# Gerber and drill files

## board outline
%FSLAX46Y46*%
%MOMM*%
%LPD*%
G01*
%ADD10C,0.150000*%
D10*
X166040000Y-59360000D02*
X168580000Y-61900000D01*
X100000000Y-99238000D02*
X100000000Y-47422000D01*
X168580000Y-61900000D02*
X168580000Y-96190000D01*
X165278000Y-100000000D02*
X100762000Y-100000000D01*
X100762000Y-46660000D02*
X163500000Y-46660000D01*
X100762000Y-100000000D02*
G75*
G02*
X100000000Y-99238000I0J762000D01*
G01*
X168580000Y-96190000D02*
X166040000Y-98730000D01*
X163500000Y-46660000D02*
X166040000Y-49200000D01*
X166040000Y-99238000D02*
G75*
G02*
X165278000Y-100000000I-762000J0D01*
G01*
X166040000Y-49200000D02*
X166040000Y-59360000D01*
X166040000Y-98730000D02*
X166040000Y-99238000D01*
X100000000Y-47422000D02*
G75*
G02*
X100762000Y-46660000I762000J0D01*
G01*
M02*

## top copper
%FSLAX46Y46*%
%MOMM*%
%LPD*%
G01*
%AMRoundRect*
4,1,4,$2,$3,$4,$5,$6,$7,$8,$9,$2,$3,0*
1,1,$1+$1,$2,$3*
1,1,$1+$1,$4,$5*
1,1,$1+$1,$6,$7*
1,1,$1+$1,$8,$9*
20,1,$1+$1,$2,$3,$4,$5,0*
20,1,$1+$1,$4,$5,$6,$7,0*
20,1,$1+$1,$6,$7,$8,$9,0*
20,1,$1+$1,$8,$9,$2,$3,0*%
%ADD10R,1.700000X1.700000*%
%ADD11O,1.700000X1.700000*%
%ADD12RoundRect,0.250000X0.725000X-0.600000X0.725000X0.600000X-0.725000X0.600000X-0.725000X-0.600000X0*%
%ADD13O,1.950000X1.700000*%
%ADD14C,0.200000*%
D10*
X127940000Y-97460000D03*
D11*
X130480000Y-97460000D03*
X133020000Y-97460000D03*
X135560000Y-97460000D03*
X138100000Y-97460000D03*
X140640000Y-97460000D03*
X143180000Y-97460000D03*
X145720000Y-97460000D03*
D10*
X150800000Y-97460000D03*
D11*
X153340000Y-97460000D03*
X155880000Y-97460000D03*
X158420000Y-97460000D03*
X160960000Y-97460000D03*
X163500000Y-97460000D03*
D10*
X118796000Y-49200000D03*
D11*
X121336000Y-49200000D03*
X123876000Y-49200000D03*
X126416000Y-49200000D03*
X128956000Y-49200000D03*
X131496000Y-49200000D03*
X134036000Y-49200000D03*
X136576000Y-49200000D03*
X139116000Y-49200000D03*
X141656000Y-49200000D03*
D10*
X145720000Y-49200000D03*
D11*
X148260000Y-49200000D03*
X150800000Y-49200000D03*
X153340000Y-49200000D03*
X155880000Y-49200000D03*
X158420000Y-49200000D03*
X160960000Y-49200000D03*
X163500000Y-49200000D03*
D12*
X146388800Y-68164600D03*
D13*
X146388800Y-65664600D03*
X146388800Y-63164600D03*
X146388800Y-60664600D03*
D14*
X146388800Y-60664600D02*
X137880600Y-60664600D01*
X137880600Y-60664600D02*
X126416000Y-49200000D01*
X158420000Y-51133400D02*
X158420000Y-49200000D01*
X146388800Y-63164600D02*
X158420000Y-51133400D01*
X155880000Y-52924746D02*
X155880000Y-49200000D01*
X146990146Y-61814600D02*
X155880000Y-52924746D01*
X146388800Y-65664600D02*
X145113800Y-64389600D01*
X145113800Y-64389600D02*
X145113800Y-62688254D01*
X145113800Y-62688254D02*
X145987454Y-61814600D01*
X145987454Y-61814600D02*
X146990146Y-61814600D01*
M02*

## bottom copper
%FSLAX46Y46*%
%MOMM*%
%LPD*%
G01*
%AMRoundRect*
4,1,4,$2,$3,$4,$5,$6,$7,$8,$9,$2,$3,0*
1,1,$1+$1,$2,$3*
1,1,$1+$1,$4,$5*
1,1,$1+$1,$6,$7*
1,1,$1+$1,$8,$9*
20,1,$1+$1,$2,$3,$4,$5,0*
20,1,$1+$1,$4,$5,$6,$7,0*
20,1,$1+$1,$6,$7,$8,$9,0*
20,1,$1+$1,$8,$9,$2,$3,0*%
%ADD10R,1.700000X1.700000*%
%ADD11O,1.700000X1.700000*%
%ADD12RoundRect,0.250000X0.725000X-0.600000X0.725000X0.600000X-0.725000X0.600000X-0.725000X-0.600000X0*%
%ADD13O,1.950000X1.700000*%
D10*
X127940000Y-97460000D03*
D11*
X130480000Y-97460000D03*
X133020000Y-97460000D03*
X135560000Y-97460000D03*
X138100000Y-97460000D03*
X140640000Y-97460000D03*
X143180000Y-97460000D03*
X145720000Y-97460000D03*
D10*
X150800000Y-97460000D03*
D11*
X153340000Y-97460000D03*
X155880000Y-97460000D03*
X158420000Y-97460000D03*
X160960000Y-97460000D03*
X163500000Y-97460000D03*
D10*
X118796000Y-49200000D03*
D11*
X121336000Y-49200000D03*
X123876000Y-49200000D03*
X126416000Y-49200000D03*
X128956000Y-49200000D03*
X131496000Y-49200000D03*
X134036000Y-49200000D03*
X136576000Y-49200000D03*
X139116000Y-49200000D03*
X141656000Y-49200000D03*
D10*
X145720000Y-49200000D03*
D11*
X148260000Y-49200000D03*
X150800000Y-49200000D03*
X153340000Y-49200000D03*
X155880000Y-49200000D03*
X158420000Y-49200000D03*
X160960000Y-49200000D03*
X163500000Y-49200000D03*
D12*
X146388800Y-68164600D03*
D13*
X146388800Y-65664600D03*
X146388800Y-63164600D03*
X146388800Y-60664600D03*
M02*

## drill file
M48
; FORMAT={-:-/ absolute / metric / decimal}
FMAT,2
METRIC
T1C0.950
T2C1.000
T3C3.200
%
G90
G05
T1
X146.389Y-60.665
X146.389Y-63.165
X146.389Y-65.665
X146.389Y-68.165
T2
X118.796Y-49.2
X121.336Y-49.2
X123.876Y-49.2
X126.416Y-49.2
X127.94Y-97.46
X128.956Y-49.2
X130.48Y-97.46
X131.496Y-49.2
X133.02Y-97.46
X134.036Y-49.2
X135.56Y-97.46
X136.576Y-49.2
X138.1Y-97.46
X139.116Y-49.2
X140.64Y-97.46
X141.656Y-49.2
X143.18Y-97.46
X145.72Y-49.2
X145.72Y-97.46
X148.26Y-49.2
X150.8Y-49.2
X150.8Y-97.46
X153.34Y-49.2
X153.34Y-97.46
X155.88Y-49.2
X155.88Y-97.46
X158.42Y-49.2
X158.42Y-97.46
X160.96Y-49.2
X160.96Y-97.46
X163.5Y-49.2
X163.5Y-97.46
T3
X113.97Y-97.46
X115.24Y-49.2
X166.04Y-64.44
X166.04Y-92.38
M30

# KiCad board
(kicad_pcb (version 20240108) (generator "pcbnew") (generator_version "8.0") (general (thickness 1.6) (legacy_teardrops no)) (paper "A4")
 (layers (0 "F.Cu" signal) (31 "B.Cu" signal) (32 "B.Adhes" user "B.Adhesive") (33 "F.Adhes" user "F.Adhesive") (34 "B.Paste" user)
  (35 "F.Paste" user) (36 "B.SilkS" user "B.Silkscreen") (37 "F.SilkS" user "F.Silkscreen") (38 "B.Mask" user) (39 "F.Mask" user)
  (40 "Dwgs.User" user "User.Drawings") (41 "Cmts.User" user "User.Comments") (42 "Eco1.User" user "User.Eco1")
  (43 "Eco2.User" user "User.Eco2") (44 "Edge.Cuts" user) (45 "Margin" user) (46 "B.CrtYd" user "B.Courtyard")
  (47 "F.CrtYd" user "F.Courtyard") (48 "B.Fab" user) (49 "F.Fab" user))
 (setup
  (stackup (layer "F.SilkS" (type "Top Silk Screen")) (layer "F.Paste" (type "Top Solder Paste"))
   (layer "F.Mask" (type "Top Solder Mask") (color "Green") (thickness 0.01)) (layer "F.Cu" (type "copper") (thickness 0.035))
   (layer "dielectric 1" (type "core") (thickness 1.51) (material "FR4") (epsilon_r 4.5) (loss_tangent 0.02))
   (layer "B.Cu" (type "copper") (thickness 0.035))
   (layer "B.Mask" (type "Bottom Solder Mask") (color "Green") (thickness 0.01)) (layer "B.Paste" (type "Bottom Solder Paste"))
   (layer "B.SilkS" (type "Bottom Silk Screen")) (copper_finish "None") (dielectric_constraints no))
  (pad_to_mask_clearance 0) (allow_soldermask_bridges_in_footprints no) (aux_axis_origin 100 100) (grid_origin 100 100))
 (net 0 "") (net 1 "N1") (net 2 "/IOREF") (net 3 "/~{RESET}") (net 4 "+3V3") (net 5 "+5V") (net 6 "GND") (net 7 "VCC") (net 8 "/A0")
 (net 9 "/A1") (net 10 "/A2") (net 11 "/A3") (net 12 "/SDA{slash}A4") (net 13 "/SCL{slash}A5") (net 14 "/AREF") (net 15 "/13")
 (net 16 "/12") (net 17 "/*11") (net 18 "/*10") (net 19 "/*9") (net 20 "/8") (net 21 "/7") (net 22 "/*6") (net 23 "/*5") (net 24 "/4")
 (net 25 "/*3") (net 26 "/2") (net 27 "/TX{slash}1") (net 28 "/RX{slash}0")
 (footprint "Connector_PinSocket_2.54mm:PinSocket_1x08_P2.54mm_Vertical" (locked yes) (layer "F.Cu") (at 127.94 97.46 90)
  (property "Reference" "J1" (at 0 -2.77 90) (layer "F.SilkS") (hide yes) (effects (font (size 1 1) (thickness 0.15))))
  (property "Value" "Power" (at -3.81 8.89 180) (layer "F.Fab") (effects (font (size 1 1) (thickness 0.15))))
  (pad "1" thru_hole rect (at 0 0 90) (size 1.7 1.7) (drill 1) (layers "*.Cu" "*.Mask") (remove_unused_layers no) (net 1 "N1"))
  (pad "2" thru_hole oval (at 0 2.54 90) (size 1.7 1.7) (drill 1) (layers "*.Cu" "*.Mask") (remove_unused_layers no) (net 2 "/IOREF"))
  (pad "3" thru_hole oval (at 0 5.08 90) (size 1.7 1.7) (drill 1) (layers "*.Cu" "*.Mask") (remove_unused_layers no) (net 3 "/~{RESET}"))
  (pad "4" thru_hole oval (at 0 7.62 90) (size 1.7 1.7) (drill 1) (layers "*.Cu" "*.Mask") (remove_unused_layers no) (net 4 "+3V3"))
  (pad "5" thru_hole oval (at 0 10.16 90) (size 1.7 1.7) (drill 1) (layers "*.Cu" "*.Mask") (remove_unused_layers no) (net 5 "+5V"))
  (pad "6" thru_hole oval (at 0 12.7 90) (size 1.7 1.7) (drill 1) (layers "*.Cu" "*.Mask") (remove_unused_layers no) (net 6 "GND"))
  (pad "7" thru_hole oval (at 0 15.24 90) (size 1.7 1.7) (drill 1) (layers "*.Cu" "*.Mask") (remove_unused_layers no) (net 6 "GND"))
  (pad "8" thru_hole oval (at 0 17.78 90) (size 1.7 1.7) (drill 1) (layers "*.Cu" "*.Mask") (remove_unused_layers no) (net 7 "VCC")))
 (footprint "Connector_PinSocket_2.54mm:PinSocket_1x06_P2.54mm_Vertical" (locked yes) (layer "F.Cu") (at 150.8 97.46 90)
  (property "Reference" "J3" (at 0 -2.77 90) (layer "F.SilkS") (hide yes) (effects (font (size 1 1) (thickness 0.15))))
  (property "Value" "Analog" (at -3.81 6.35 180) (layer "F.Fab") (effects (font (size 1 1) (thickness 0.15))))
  (pad "1" thru_hole rect (at 0 0 90) (size 1.7 1.7) (drill 1) (layers "*.Cu" "*.Mask") (remove_unused_layers no) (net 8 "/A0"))
  (pad "2" thru_hole oval (at 0 2.54 90) (size 1.7 1.7) (drill 1) (layers "*.Cu" "*.Mask") (remove_unused_layers no) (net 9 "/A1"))
  (pad "3" thru_hole oval (at 0 5.08 90) (size 1.7 1.7) (drill 1) (layers "*.Cu" "*.Mask") (remove_unused_layers no) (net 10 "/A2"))
  (pad "4" thru_hole oval (at 0 7.62 90) (size 1.7 1.7) (drill 1) (layers "*.Cu" "*.Mask") (remove_unused_layers no) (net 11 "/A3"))
  (pad "5" thru_hole oval (at 0 10.16 90) (size 1.7 1.7) (drill 1) (layers "*.Cu" "*.Mask") (remove_unused_layers no)
   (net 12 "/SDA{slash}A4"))
  (pad "6" thru_hole oval (at 0 12.7 90) (size 1.7 1.7) (drill 1) (layers "*.Cu" "*.Mask") (remove_unused_layers no)
   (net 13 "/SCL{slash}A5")))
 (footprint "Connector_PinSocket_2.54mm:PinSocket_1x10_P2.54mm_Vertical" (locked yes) (layer "F.Cu") (at 118.796 49.2 90)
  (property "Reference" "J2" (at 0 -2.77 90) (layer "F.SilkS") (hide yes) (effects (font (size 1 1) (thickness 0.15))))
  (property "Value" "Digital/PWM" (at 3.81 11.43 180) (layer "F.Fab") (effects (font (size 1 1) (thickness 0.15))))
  (pad "1" thru_hole rect (at 0 0 90) (size 1.7 1.7) (drill 1) (layers "*.Cu" "*.Mask") (remove_unused_layers no) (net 13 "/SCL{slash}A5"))
  (pad "2" thru_hole oval (at 0 2.54 90) (size 1.7 1.7) (drill 1) (layers "*.Cu" "*.Mask") (remove_unused_layers no)
   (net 12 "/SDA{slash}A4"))
  (pad "3" thru_hole oval (at 0 5.08 90) (size 1.7 1.7) (drill 1) (layers "*.Cu" "*.Mask") (remove_unused_layers no) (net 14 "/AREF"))
  (pad "4" thru_hole oval (at 0 7.62 90) (size 1.7 1.7) (drill 1) (layers "*.Cu" "*.Mask") (remove_unused_layers no) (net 6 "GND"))
  (pad "5" thru_hole oval (at 0 10.16 90) (size 1.7 1.7) (drill 1) (layers "*.Cu" "*.Mask") (remove_unused_layers no) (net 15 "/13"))
  (pad "6" thru_hole oval (at 0 12.7 90) (size 1.7 1.7) (drill 1) (layers "*.Cu" "*.Mask") (remove_unused_layers no) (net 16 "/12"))
  (pad "7" thru_hole oval (at 0 15.24 90) (size 1.7 1.7) (drill 1) (layers "*.Cu" "*.Mask") (remove_unused_layers no) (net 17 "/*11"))
  (pad "8" thru_hole oval (at 0 17.78 90) (size 1.7 1.7) (drill 1) (layers "*.Cu" "*.Mask") (remove_unused_layers no) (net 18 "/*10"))
  (pad "9" thru_hole oval (at 0 20.32 90) (size 1.7 1.7) (drill 1) (layers "*.Cu" "*.Mask") (remove_unused_layers no) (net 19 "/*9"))
  (pad "10" thru_hole oval (at 0 22.86 90) (size 1.7 1.7) (drill 1) (layers "*.Cu" "*.Mask") (remove_unused_layers no) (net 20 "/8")))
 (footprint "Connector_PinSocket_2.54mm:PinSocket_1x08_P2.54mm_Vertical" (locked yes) (layer "F.Cu") (at 145.72 49.2 90)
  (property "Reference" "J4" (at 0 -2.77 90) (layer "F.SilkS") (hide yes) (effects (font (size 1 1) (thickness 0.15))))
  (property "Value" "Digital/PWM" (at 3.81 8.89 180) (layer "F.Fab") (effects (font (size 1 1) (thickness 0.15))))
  (pad "1" thru_hole rect (at 0 0 90) (size 1.7 1.7) (drill 1) (layers "*.Cu" "*.Mask") (remove_unused_layers no) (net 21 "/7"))
  (pad "2" thru_hole oval (at 0 2.54 90) (size 1.7 1.7) (drill 1) (layers "*.Cu" "*.Mask") (remove_unused_layers no) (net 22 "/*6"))
  (pad "3" thru_hole oval (at 0 5.08 90) (size 1.7 1.7) (drill 1) (layers "*.Cu" "*.Mask") (remove_unused_layers no) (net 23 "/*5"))
  (pad "4" thru_hole oval (at 0 7.62 90) (size 1.7 1.7) (drill 1) (layers "*.Cu" "*.Mask") (remove_unused_layers no) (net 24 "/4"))
  (pad "5" thru_hole oval (at 0 10.16 90) (size 1.7 1.7) (drill 1) (layers "*.Cu" "*.Mask") (remove_unused_layers no) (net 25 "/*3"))
  (pad "6" thru_hole oval (at 0 12.7 90) (size 1.7 1.7) (drill 1) (layers "*.Cu" "*.Mask") (remove_unused_layers no) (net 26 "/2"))
  (pad "7" thru_hole oval (at 0 15.24 90) (size 1.7 1.7) (drill 1) (layers "*.Cu" "*.Mask") (remove_unused_layers no) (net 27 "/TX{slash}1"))
  (pad "8" thru_hole oval (at 0 17.78 90) (size 1.7 1.7) (drill 1) (layers "*.Cu" "*.Mask") (remove_unused_layers no) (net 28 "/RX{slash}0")))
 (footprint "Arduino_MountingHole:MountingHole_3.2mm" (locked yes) (layer "F.Cu") (at 115.24 49.2)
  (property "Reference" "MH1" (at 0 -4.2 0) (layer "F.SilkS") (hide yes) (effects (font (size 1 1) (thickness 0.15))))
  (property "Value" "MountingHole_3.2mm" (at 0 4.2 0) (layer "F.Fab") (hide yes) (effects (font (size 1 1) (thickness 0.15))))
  (pad "" np_thru_hole circle (at 0 0) (size 3.2 3.2) (drill 3.2) (layers "*.Cu" "*.Mask")))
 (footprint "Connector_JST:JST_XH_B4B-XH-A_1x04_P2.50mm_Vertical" (layer "F.Cu") (at 146.3888 68.1646 90)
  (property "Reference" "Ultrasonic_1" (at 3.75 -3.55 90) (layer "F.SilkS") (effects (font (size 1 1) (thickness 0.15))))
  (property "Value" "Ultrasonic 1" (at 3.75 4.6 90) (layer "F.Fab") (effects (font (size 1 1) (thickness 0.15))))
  (pad "1" thru_hole roundrect (at 0 0 90) (size 1.7 1.95) (drill 0.95) (layers "*.Cu" "*.Mask") (remove_unused_layers no)
   (roundrect_rratio 0.147059) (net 7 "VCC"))
  (pad "2" thru_hole oval (at 2.5 0 90) (size 1.7 1.95) (drill 0.95) (layers "*.Cu" "*.Mask") (remove_unused_layers no) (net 25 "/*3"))
  (pad "3" thru_hole oval (at 5 0 90) (size 1.7 1.95) (drill 0.95) (layers "*.Cu" "*.Mask") (remove_unused_layers no) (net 26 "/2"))
  (pad "4" thru_hole oval (at 7.5 0 90) (size 1.7 1.95) (drill 0.95) (layers "*.Cu" "*.Mask") (remove_unused_layers no) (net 6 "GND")))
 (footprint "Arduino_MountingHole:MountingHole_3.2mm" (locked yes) (layer "F.Cu") (at 113.97 97.46)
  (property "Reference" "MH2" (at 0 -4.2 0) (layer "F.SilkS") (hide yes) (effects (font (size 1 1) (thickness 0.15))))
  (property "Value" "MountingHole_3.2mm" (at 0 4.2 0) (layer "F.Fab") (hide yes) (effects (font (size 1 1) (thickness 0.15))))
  (pad "" np_thru_hole circle (at 0 0) (size 3.2 3.2) (drill 3.2) (layers "*.Cu" "*.Mask")))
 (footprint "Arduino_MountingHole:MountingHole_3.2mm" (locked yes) (layer "F.Cu") (at 166.04 64.44)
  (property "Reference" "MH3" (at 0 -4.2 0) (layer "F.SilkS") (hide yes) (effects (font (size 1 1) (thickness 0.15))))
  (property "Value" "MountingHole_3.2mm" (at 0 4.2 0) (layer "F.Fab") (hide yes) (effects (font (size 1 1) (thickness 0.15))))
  (pad "" np_thru_hole circle (at 0 0) (size 3.2 3.2) (drill 3.2) (layers "*.Cu" "*.Mask")))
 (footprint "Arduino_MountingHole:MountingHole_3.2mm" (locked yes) (layer "F.Cu") (at 166.04 92.38)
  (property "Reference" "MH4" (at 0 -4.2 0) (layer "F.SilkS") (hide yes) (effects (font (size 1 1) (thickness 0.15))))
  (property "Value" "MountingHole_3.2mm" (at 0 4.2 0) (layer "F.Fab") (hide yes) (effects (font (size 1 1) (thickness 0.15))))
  (pad "" np_thru_hole circle (at 0 0) (size 3.2 3.2) (drill 3.2) (layers "*.Cu" "*.Mask")))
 (gr_line (start 166.04 59.36) (end 168.58 61.9) (stroke (width 0.15) (type solid)) (layer "Edge.Cuts"))
 (gr_line (start 100 99.238) (end 100 47.422) (stroke (width 0.15) (type solid)) (layer "Edge.Cuts"))
 (gr_line (start 168.58 61.9) (end 168.58 96.19) (stroke (width 0.15) (type solid)) (layer "Edge.Cuts"))
 (gr_line (start 165.278 100) (end 100.762 100) (stroke (width 0.15) (type solid)) (layer "Edge.Cuts"))
 (gr_line (start 100.762 46.66) (end 163.5 46.66) (stroke (width 0.15) (type solid)) (layer "Edge.Cuts"))
 (gr_arc (start 100.762 100) (mid 100.223185 99.776815) (end 100 99.238) (stroke (width 0.15) (type solid)) (layer "Edge.Cuts"))
 (gr_line (start 168.58 96.19) (end 166.04 98.73) (stroke (width 0.15) (type solid)) (layer "Edge.Cuts"))
 (gr_line (start 163.5 46.66) (end 166.04 49.2) (stroke (width 0.15) (type solid)) (layer "Edge.Cuts"))
 (gr_arc (start 166.04 99.238) (mid 165.816815 99.776815) (end 165.278 100) (stroke (width 0.15) (type solid)) (layer "Edge.Cuts"))
 (gr_line (start 166.04 49.2) (end 166.04 59.36) (stroke (width 0.15) (type solid)) (layer "Edge.Cuts"))
 (gr_line (start 166.04 98.73) (end 166.04 99.238) (stroke (width 0.15) (type solid)) (layer "Edge.Cuts"))
 (gr_arc (start 100 47.422) (mid 100.223185 46.883185) (end 100.762 46.66) (stroke (width 0.15) (type solid)) (layer "Edge.Cuts"))
 (segment (start 146.3888 60.6646) (end 137.8806 60.6646) (width 0.2) (layer "F.Cu") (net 6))
 (segment (start 137.8806 60.6646) (end 126.416 49.2) (width 0.2) (layer "F.Cu") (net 6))
 (segment (start 158.42 51.1334) (end 158.42 49.2) (width 0.2) (layer "F.Cu") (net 26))
 (segment (start 146.3888 63.1646) (end 158.42 51.1334) (width 0.2) (layer "F.Cu") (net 26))
 (segment (start 155.88 52.924746) (end 155.88 49.2) (width 0.2) (layer "F.Cu") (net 25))
 (segment (start 146.990146 61.8146) (end 155.88 52.924746) (width 0.2) (layer "F.Cu") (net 25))
 (segment (start 146.3888 65.6646) (end 145.1138 64.3896) (width 0.2) (layer "F.Cu") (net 25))
 (segment (start 145.1138 64.3896) (end 145.1138 62.688254) (width 0.2) (layer "F.Cu") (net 25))
 (segment (start 145.1138 62.688254) (end 145.987454 61.8146) (width 0.2) (layer "F.Cu") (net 25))
 (segment (start 145.987454 61.8146) (end 146.990146 61.8146) (width 0.2) (layer "F.Cu") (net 25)))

